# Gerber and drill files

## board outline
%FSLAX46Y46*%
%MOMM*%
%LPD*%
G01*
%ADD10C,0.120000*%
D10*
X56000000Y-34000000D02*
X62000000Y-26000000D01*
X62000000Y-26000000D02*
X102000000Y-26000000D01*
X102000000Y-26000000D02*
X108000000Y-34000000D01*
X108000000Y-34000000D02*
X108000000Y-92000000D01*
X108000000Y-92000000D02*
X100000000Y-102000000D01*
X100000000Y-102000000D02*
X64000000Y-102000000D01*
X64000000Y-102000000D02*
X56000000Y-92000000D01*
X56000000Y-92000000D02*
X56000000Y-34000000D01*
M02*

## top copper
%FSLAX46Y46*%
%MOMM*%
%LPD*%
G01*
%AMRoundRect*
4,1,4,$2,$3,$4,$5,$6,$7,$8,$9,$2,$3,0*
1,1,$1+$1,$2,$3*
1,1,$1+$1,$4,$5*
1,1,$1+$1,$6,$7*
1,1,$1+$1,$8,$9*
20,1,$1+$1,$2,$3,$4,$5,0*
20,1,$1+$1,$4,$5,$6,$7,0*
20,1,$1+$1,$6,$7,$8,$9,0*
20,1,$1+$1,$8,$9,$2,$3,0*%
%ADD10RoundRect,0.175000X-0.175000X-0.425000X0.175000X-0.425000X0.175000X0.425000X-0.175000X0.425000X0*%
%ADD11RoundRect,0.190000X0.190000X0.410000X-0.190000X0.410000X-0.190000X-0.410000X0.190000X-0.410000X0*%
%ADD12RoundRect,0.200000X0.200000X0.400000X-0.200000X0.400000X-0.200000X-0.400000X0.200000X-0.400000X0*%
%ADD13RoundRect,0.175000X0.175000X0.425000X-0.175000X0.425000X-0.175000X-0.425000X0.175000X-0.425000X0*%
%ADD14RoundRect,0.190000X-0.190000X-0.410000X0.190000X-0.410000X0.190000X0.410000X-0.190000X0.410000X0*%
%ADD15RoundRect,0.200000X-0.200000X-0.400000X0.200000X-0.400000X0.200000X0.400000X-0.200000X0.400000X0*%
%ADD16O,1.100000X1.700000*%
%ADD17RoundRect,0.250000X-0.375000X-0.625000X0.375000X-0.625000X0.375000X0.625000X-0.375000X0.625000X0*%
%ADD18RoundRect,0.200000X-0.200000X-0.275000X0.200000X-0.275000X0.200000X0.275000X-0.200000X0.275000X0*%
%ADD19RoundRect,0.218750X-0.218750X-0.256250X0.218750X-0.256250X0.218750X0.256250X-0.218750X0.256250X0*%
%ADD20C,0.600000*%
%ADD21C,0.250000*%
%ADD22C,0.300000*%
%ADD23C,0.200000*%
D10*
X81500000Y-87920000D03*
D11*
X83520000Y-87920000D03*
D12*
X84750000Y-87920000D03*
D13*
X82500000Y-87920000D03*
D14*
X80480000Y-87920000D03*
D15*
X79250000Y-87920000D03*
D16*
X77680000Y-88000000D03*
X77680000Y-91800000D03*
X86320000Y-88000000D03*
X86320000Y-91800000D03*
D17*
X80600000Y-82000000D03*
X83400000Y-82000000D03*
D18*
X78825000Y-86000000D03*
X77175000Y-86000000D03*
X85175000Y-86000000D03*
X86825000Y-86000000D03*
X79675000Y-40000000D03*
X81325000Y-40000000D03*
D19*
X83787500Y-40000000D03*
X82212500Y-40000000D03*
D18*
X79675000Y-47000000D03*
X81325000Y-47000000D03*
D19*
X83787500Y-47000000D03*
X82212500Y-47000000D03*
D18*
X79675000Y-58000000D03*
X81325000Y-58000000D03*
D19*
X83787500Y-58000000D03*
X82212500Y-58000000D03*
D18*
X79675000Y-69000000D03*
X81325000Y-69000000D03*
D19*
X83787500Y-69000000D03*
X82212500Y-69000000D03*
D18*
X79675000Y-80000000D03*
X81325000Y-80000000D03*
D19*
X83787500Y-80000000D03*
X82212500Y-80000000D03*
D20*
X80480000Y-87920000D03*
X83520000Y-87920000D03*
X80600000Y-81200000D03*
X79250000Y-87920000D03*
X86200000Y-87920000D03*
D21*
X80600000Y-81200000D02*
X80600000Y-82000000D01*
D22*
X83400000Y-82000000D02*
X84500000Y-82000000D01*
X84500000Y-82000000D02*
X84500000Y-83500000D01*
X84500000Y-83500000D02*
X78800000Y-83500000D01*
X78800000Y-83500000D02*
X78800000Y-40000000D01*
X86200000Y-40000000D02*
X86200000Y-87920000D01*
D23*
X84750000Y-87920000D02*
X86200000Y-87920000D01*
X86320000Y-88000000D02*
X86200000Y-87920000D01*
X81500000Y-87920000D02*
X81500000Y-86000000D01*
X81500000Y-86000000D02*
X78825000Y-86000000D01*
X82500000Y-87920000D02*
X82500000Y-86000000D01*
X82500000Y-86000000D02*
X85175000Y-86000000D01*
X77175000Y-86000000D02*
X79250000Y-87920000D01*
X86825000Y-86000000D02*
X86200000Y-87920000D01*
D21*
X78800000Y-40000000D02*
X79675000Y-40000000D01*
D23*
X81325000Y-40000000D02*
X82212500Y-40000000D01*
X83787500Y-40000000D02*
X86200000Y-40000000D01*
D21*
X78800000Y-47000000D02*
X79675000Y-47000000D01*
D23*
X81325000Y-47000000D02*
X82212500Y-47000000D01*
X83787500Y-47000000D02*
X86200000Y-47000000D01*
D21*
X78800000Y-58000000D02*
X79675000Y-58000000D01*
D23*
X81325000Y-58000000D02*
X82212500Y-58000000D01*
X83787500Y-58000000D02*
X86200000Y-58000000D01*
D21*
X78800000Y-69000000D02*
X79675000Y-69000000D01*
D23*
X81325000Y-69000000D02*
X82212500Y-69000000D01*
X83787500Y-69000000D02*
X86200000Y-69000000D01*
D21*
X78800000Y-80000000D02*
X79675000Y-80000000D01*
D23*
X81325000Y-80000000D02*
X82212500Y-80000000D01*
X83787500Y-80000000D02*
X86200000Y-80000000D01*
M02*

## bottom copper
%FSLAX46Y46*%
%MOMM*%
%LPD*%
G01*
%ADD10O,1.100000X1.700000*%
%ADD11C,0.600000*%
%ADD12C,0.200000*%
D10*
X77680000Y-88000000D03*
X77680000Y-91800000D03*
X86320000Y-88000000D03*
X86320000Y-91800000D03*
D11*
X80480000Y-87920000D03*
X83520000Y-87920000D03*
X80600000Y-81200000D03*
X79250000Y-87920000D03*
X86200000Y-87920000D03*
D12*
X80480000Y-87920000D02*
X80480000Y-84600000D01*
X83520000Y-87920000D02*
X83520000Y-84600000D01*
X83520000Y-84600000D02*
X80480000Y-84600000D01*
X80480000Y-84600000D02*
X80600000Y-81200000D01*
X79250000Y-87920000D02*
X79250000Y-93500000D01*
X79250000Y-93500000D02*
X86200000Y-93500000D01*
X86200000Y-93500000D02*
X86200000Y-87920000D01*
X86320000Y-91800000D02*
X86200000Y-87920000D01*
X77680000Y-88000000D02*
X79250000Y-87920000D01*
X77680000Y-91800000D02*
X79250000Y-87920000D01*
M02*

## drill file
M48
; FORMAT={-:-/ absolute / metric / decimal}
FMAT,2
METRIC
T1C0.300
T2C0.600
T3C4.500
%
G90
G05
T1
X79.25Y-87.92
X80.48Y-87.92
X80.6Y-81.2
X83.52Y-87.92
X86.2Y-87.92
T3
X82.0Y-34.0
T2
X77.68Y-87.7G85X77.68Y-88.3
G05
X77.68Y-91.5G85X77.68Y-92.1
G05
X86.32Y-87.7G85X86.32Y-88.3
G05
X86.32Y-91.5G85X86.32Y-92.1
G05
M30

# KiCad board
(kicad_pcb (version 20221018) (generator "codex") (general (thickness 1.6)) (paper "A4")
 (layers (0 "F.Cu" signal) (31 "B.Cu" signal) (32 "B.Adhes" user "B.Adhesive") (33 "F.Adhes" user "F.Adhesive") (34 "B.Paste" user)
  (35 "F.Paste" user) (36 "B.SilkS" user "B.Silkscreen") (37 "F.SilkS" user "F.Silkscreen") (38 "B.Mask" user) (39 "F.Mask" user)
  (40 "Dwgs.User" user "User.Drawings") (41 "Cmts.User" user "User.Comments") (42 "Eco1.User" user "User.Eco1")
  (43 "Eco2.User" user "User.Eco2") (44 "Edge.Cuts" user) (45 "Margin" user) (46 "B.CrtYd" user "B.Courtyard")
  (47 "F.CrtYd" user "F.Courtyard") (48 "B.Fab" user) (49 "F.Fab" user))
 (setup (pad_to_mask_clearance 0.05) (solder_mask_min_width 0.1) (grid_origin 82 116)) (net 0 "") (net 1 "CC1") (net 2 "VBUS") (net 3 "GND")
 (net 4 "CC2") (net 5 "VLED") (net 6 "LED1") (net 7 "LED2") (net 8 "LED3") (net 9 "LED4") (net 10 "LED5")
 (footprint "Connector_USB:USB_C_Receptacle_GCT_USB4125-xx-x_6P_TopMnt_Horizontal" (layer "F.Cu") (at 82 91)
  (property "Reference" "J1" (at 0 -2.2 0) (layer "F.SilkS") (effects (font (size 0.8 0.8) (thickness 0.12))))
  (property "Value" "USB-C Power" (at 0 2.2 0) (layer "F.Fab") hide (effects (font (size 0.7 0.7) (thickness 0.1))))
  (pad "A5" smd roundrect (at -0.5 -3.08) (size 0.7 1.2) (layers "F.Cu" "F.Paste" "F.Mask") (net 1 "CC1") (roundrect_rratio 0.25))
  (pad "A9" smd roundrect (at 1.52 -3.08 180) (size 0.76 1.2) (layers "F.Cu" "F.Paste" "F.Mask") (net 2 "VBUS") (roundrect_rratio 0.25))
  (pad "A12" smd roundrect (at 2.75 -3.08 180) (size 0.8 1.2) (layers "F.Cu" "F.Paste" "F.Mask") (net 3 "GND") (roundrect_rratio 0.25))
  (pad "B5" smd roundrect (at 0.5 -3.08 180) (size 0.7 1.2) (layers "F.Cu" "F.Paste" "F.Mask") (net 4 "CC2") (roundrect_rratio 0.25))
  (pad "B9" smd roundrect (at -1.52 -3.08) (size 0.76 1.2) (layers "F.Cu" "F.Paste" "F.Mask") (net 2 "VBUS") (roundrect_rratio 0.25))
  (pad "B12" smd roundrect (at -2.75 -3.08) (size 0.8 1.2) (layers "F.Cu" "F.Paste" "F.Mask") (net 3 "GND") (roundrect_rratio 0.25))
  (pad "SH" thru_hole oval (at -4.32 -3) (size 1.1 1.7) (drill oval 0.6 1.2) (layers "*.Cu" "*.Mask") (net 3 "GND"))
  (pad "SH" thru_hole oval (at -4.32 0.8) (size 1.1 1.7) (drill oval 0.6 1.2) (layers "*.Cu" "*.Mask") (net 3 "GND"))
  (pad "SH" thru_hole oval (at 4.32 -3) (size 1.1 1.7) (drill oval 0.6 1.2) (layers "*.Cu" "*.Mask") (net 3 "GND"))
  (pad "SH" thru_hole oval (at 4.32 0.8) (size 1.1 1.7) (drill oval 0.6 1.2) (layers "*.Cu" "*.Mask") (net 3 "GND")))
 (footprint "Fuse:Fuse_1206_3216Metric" (layer "F.Cu") (at 82 82)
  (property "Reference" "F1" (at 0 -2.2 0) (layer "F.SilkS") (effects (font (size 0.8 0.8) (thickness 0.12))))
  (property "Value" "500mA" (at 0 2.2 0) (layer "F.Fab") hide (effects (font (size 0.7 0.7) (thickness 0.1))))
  (pad "1" smd roundrect (at -1.4 0) (size 1.25 1.75) (layers "F.Cu" "F.Paste" "F.Mask") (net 2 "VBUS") (roundrect_rratio 0.2))
  (pad "2" smd roundrect (at 1.4 0) (size 1.25 1.75) (layers "F.Cu" "F.Paste" "F.Mask") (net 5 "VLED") (roundrect_rratio 0.2)))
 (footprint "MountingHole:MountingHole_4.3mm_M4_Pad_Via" (layer "F.Cu") (at 82 34)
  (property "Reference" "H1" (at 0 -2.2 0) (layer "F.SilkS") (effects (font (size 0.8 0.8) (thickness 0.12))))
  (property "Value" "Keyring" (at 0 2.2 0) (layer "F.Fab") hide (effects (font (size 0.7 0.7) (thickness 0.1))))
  (pad "1" np_thru_hole circle (at 0 0) (size 4.5 4.5) (drill 4.5) (layers "*.Cu" "*.Mask")))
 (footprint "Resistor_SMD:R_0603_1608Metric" (layer "F.Cu") (at 78 86 180)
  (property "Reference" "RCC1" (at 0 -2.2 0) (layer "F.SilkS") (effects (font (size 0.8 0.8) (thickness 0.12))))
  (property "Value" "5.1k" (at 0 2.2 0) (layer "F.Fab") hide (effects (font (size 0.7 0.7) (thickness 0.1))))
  (pad "1" smd roundrect (at -0.825 0) (size 0.8 0.95) (layers "F.Cu" "F.Paste" "F.Mask") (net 1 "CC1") (roundrect_rratio 0.25))
  (pad "2" smd roundrect (at 0.825 0) (size 0.8 0.95) (layers "F.Cu" "F.Paste" "F.Mask") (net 3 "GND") (roundrect_rratio 0.25)))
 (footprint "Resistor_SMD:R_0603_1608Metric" (layer "F.Cu") (at 86 86)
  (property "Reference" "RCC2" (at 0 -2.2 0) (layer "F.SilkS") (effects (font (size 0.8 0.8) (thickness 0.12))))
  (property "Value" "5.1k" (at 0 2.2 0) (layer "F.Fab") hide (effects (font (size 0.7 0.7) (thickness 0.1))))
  (pad "1" smd roundrect (at -0.825 0) (size 0.8 0.95) (layers "F.Cu" "F.Paste" "F.Mask") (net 4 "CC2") (roundrect_rratio 0.25))
  (pad "2" smd roundrect (at 0.825 0) (size 0.8 0.95) (layers "F.Cu" "F.Paste" "F.Mask") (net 3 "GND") (roundrect_rratio 0.25)))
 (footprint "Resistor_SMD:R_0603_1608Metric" (layer "F.Cu") (at 80.5 40 0)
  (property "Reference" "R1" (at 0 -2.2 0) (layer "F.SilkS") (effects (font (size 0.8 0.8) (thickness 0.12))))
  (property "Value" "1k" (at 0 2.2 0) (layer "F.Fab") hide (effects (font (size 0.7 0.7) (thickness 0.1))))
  (pad "1" smd roundrect (at -0.825 0) (size 0.8 0.95) (layers "F.Cu" "F.Paste" "F.Mask") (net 5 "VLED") (roundrect_rratio 0.25))
  (pad "2" smd roundrect (at 0.825 0) (size 0.8 0.95) (layers "F.Cu" "F.Paste" "F.Mask") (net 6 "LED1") (roundrect_rratio 0.25)))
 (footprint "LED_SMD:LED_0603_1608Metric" (layer "F.Cu") (at 83 40 180)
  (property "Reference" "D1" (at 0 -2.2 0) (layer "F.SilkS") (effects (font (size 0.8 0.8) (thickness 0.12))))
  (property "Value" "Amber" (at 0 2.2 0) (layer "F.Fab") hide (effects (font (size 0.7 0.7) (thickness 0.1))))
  (pad "1" smd roundrect (at -0.7875 0) (size 0.875 0.95) (layers "F.Cu" "F.Paste" "F.Mask") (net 3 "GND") (roundrect_rratio 0.25))
  (pad "2" smd roundrect (at 0.7875 0) (size 0.875 0.95) (layers "F.Cu" "F.Paste" "F.Mask") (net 6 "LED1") (roundrect_rratio 0.25)))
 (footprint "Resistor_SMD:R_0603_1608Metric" (layer "F.Cu") (at 80.5 47 0)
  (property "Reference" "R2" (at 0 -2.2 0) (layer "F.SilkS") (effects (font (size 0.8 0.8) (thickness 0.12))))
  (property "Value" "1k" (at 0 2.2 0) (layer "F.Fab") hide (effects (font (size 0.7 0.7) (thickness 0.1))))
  (pad "1" smd roundrect (at -0.825 0) (size 0.8 0.95) (layers "F.Cu" "F.Paste" "F.Mask") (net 5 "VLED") (roundrect_rratio 0.25))
  (pad "2" smd roundrect (at 0.825 0) (size 0.8 0.95) (layers "F.Cu" "F.Paste" "F.Mask") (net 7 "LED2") (roundrect_rratio 0.25)))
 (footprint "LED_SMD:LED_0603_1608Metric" (layer "F.Cu") (at 83 47 180)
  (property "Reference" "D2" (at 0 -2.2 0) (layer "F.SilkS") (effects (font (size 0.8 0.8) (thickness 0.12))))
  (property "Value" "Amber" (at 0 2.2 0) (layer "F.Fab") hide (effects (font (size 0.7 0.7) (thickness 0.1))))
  (pad "1" smd roundrect (at -0.7875 0) (size 0.875 0.95) (layers "F.Cu" "F.Paste" "F.Mask") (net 3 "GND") (roundrect_rratio 0.25))
  (pad "2" smd roundrect (at 0.7875 0) (size 0.875 0.95) (layers "F.Cu" "F.Paste" "F.Mask") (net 7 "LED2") (roundrect_rratio 0.25)))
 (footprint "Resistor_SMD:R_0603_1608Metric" (layer "F.Cu") (at 80.5 58 0)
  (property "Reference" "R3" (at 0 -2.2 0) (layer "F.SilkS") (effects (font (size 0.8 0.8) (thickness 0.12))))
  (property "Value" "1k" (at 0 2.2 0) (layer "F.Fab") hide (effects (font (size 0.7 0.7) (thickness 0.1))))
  (pad "1" smd roundrect (at -0.825 0) (size 0.8 0.95) (layers "F.Cu" "F.Paste" "F.Mask") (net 5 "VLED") (roundrect_rratio 0.25))
  (pad "2" smd roundrect (at 0.825 0) (size 0.8 0.95) (layers "F.Cu" "F.Paste" "F.Mask") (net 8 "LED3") (roundrect_rratio 0.25)))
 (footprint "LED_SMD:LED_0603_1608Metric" (layer "F.Cu") (at 83 58 180)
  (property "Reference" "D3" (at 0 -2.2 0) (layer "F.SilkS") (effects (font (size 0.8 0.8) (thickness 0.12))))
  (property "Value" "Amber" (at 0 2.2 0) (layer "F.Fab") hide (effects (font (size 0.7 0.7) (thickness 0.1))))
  (pad "1" smd roundrect (at -0.7875 0) (size 0.875 0.95) (layers "F.Cu" "F.Paste" "F.Mask") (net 3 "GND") (roundrect_rratio 0.25))
  (pad "2" smd roundrect (at 0.7875 0) (size 0.875 0.95) (layers "F.Cu" "F.Paste" "F.Mask") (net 8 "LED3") (roundrect_rratio 0.25)))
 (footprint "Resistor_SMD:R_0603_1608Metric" (layer "F.Cu") (at 80.5 69 0)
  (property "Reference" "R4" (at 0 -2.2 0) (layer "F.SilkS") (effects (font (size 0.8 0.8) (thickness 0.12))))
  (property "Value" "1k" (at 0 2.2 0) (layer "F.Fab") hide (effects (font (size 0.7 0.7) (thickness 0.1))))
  (pad "1" smd roundrect (at -0.825 0) (size 0.8 0.95) (layers "F.Cu" "F.Paste" "F.Mask") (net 5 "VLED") (roundrect_rratio 0.25))
  (pad "2" smd roundrect (at 0.825 0) (size 0.8 0.95) (layers "F.Cu" "F.Paste" "F.Mask") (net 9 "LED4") (roundrect_rratio 0.25)))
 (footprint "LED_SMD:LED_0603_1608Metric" (layer "F.Cu") (at 83 69 180)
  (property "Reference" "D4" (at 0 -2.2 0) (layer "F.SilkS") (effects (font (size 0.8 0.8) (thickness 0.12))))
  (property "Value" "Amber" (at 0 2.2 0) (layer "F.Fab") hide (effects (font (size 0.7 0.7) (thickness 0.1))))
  (pad "1" smd roundrect (at -0.7875 0) (size 0.875 0.95) (layers "F.Cu" "F.Paste" "F.Mask") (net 3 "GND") (roundrect_rratio 0.25))
  (pad "2" smd roundrect (at 0.7875 0) (size 0.875 0.95) (layers "F.Cu" "F.Paste" "F.Mask") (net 9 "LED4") (roundrect_rratio 0.25)))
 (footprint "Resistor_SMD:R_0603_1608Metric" (layer "F.Cu") (at 80.5 80 0)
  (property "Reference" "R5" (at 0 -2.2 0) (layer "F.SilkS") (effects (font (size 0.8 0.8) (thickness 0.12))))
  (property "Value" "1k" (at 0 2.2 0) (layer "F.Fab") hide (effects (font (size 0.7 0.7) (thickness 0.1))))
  (pad "1" smd roundrect (at -0.825 0) (size 0.8 0.95) (layers "F.Cu" "F.Paste" "F.Mask") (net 5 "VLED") (roundrect_rratio 0.25))
  (pad "2" smd roundrect (at 0.825 0) (size 0.8 0.95) (layers "F.Cu" "F.Paste" "F.Mask") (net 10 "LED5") (roundrect_rratio 0.25)))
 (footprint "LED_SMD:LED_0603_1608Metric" (layer "F.Cu") (at 83 80 180)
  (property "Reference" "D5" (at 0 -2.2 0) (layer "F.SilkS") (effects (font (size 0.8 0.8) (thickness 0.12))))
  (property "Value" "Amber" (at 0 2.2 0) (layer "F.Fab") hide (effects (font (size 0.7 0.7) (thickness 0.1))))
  (pad "1" smd roundrect (at -0.7875 0) (size 0.875 0.95) (layers "F.Cu" "F.Paste" "F.Mask") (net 3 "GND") (roundrect_rratio 0.25))
  (pad "2" smd roundrect (at 0.7875 0) (size 0.875 0.95) (layers "F.Cu" "F.Paste" "F.Mask") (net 10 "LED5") (roundrect_rratio 0.25)))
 (gr_line (start 56 34) (end 62 26) (stroke (width 0.12) (type solid)) (layer "Edge.Cuts"))
 (gr_line (start 62 26) (end 102 26) (stroke (width 0.12) (type solid)) (layer "Edge.Cuts"))
 (gr_line (start 102 26) (end 108 34) (stroke (width 0.12) (type solid)) (layer "Edge.Cuts"))
 (gr_line (start 108 34) (end 108 92) (stroke (width 0.12) (type solid)) (layer "Edge.Cuts"))
 (gr_line (start 108 92) (end 100 102) (stroke (width 0.12) (type solid)) (layer "Edge.Cuts"))
 (gr_line (start 100 102) (end 64 102) (stroke (width 0.12) (type solid)) (layer "Edge.Cuts"))
 (gr_line (start 64 102) (end 56 92) (stroke (width 0.12) (type solid)) (layer "Edge.Cuts"))
 (gr_line (start 56 92) (end 56 34) (stroke (width 0.12) (type solid)) (layer "Edge.Cuts"))
 (via (at 80.48 87.92) (size 0.6) (drill 0.3) (layers "F.Cu" "B.Cu") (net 2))
 (via (at 83.52 87.92) (size 0.6) (drill 0.3) (layers "F.Cu" "B.Cu") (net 2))
 (via (at 80.6 81.2) (size 0.6) (drill 0.3) (layers "F.Cu" "B.Cu") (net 2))
 (via (at 79.25 87.92) (size 0.6) (drill 0.3) (layers "F.Cu" "B.Cu") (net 3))
 (via (at 86.2 87.92) (size 0.6) (drill 0.3) (layers "F.Cu" "B.Cu") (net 3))
 (segment (start 80.6 81.2) (end 80.6 82.0) (width 0.25) (layer "F.Cu") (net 2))
 (segment (start 80.48 87.92) (end 80.48 84.6) (width 0.20) (layer "B.Cu") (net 2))
 (segment (start 83.52 87.92) (end 83.52 84.6) (width 0.20) (layer "B.Cu") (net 2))
 (segment (start 83.52 84.6) (end 80.48 84.6) (width 0.20) (layer "B.Cu") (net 2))
 (segment (start 80.48 84.6) (end 80.6 81.2) (width 0.20) (layer "B.Cu") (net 2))
 (segment (start 83.4 82.0) (end 84.5 82.0) (width 0.30) (layer "F.Cu") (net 5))
 (segment (start 84.5 82.0) (end 84.5 83.5) (width 0.30) (layer "F.Cu") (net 5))
 (segment (start 84.5 83.5) (end 78.8 83.5) (width 0.30) (layer "F.Cu") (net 5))
 (segment (start 78.8 83.5) (end 78.8 40.0) (width 0.30) (layer "F.Cu") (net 5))
 (segment (start 86.2 40.0) (end 86.2 87.92) (width 0.30) (layer "F.Cu") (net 3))
 (segment (start 84.75 87.92) (end 86.2 87.92) (width 0.20) (layer "F.Cu") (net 3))
 (segment (start 79.25 87.92) (end 79.25 93.5) (width 0.20) (layer "B.Cu") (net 3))
 (segment (start 79.25 93.5) (end 86.2 93.5) (width 0.20) (layer "B.Cu") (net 3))
 (segment (start 86.2 93.5) (end 86.2 87.92) (width 0.20) (layer "B.Cu") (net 3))
 (segment (start 86.32 88.0) (end 86.2 87.92) (width 0.20) (layer "F.Cu") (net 3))
 (segment (start 86.32 91.8) (end 86.2 87.92) (width 0.20) (layer "B.Cu") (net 3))
 (segment (start 77.68 88.0) (end 79.25 87.92) (width 0.20) (layer "B.Cu") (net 3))
 (segment (start 77.68 91.8) (end 79.25 87.92) (width 0.20) (layer "B.Cu") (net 3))
 (segment (start 81.5 87.92) (end 81.5 86.0) (width 0.20) (layer "F.Cu") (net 1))
 (segment (start 81.5 86.0) (end 78.825 86.0) (width 0.20) (layer "F.Cu") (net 1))
 (segment (start 82.5 87.92) (end 82.5 86.0) (width 0.20) (layer "F.Cu") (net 4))
 (segment (start 82.5 86.0) (end 85.175 86.0) (width 0.20) (layer "F.Cu") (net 4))
 (segment (start 77.175 86.0) (end 79.25 87.92) (width 0.20) (layer "F.Cu") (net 3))
 (segment (start 86.825 86.0) (end 86.2 87.92) (width 0.20) (layer "F.Cu") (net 3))
 (segment (start 78.8 40.0) (end 79.675 40.0) (width 0.25) (layer "F.Cu") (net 5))
 (segment (start 81.325 40.0) (end 82.2125 40.0) (width 0.20) (layer "F.Cu") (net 6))
 (segment (start 83.7875 40.0) (end 86.2 40.0) (width 0.20) (layer "F.Cu") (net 3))
 (segment (start 78.8 47.0) (end 79.675 47.0) (width 0.25) (layer "F.Cu") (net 5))
 (segment (start 81.325 47.0) (end 82.2125 47.0) (width 0.20) (layer "F.Cu") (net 7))
 (segment (start 83.7875 47.0) (end 86.2 47.0) (width 0.20) (layer "F.Cu") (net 3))
 (segment (start 78.8 58.0) (end 79.675 58.0) (width 0.25) (layer "F.Cu") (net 5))
 (segment (start 81.325 58.0) (end 82.2125 58.0) (width 0.20) (layer "F.Cu") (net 8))
 (segment (start 83.7875 58.0) (end 86.2 58.0) (width 0.20) (layer "F.Cu") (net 3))
 (segment (start 78.8 69.0) (end 79.675 69.0) (width 0.25) (layer "F.Cu") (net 5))
 (segment (start 81.325 69.0) (end 82.2125 69.0) (width 0.20) (layer "F.Cu") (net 9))
 (segment (start 83.7875 69.0) (end 86.2 69.0) (width 0.20) (layer "F.Cu") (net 3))
 (segment (start 78.8 80.0) (end 79.675 80.0) (width 0.25) (layer "F.Cu") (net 5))
 (segment (start 81.325 80.0) (end 82.2125 80.0) (width 0.20) (layer "F.Cu") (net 10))
 (segment (start 83.7875 80.0) (end 86.2 80.0) (width 0.20) (layer "F.Cu") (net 3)))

